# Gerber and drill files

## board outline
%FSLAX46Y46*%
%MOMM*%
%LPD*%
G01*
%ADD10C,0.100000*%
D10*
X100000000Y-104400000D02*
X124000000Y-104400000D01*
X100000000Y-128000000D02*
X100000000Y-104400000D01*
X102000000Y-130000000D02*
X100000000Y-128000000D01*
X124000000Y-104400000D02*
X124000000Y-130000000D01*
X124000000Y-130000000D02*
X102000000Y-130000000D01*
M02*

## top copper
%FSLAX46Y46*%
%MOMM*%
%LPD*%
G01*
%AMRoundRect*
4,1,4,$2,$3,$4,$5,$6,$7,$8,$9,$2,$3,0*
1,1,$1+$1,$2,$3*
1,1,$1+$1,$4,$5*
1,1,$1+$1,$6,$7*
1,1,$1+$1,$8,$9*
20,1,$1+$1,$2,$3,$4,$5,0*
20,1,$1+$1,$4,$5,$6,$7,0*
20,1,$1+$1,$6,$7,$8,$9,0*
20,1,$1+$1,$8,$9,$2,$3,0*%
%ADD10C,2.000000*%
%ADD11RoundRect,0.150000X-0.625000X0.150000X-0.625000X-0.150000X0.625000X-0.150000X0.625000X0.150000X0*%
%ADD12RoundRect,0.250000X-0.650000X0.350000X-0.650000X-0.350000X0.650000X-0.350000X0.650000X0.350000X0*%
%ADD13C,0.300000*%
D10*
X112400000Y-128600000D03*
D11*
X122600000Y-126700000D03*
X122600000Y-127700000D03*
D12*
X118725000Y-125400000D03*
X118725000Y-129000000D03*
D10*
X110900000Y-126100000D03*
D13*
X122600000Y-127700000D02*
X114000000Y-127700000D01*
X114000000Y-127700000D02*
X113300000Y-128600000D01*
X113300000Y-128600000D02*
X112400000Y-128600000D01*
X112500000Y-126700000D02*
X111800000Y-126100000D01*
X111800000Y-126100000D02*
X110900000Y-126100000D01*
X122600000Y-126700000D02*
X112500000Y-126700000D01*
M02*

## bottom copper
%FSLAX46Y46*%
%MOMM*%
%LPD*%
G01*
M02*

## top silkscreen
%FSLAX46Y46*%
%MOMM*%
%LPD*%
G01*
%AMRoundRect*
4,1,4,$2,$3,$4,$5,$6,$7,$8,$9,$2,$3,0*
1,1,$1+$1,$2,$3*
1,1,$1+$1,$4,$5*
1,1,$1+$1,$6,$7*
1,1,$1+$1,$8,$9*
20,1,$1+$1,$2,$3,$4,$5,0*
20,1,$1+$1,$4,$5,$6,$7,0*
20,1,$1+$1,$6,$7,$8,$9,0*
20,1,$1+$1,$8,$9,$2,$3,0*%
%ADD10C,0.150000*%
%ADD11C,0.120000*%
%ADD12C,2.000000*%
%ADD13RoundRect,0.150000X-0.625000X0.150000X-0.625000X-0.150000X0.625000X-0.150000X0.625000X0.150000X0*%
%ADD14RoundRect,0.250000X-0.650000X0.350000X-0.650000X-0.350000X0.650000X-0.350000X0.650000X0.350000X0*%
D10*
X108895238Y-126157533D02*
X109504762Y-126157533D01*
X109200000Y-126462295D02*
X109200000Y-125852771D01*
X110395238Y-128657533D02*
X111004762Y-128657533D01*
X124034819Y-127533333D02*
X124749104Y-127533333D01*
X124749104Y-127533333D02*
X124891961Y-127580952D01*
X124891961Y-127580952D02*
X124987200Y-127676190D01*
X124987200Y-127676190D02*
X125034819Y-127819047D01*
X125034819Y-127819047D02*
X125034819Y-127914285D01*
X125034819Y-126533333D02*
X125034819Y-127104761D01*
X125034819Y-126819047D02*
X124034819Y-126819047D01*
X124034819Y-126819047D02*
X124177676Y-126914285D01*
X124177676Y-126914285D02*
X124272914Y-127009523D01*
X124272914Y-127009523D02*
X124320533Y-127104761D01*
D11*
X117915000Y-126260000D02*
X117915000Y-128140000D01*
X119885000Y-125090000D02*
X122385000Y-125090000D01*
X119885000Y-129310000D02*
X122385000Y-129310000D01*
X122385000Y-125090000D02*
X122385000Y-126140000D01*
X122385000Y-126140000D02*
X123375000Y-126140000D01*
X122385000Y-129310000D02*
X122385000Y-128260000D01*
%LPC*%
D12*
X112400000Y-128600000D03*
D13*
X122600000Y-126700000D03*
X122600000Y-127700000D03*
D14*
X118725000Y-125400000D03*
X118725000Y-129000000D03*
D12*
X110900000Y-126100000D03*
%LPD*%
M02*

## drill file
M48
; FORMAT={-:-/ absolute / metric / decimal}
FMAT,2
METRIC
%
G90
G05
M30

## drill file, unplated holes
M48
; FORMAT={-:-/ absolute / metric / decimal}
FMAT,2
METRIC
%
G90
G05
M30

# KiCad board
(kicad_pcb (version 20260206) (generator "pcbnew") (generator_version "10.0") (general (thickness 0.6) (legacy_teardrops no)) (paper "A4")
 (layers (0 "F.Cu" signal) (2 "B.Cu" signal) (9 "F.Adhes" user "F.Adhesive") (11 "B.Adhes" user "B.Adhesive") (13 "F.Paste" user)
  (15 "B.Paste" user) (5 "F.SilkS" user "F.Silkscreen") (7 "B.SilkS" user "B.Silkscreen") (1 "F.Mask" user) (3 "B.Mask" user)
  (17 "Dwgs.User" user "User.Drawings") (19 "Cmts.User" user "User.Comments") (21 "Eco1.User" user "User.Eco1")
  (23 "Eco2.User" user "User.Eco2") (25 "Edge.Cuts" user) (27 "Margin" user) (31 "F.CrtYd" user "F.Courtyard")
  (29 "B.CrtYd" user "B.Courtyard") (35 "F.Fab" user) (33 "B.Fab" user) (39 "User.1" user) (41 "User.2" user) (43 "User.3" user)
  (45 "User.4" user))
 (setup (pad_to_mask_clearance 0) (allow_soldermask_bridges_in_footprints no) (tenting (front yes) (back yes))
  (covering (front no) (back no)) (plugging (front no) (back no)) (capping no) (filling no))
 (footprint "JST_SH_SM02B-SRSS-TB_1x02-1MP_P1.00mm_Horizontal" (layer "F.Cu") (at 120.6 127.2 -90)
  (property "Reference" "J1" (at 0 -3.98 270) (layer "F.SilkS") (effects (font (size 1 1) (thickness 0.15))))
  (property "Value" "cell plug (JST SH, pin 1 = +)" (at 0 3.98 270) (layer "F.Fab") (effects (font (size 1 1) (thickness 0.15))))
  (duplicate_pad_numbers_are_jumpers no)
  (fp_line (start -0.94 2.685) (end 0.94 2.685) (stroke (width 0.12) (type solid)) (layer "F.SilkS"))
  (fp_line (start -2.11 0.715) (end -2.11 -1.785) (stroke (width 0.12) (type solid)) (layer "F.SilkS"))
  (fp_line (start 2.11 0.715) (end 2.11 -1.785) (stroke (width 0.12) (type solid)) (layer "F.SilkS"))
  (fp_line (start -2.11 -1.785) (end -1.06 -1.785) (stroke (width 0.12) (type solid)) (layer "F.SilkS"))
  (fp_line (start -1.06 -1.785) (end -1.06 -2.775) (stroke (width 0.12) (type solid)) (layer "F.SilkS"))
  (fp_line (start 2.11 -1.785) (end 1.06 -1.785) (stroke (width 0.12) (type solid)) (layer "F.SilkS"))
  (pad "1" smd roundrect (at -0.5 -2 270) (size 0.6 1.55) (layers "F.Cu" "F.Mask" "F.Paste") (roundrect_rratio 0.25) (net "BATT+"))
  (pad "2" smd roundrect (at 0.5 -2 270) (size 0.6 1.55) (layers "F.Cu" "F.Mask" "F.Paste") (roundrect_rratio 0.25) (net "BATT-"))
  (pad "MP" smd roundrect (at -1.8 1.875 270) (size 1.2 1.8) (layers "F.Cu" "F.Mask" "F.Paste") (roundrect_rratio 0.208333))
  (pad "MP" smd roundrect (at 1.8 1.875 270) (size 1.2 1.8) (layers "F.Cu" "F.Mask" "F.Paste") (roundrect_rratio 0.208333)))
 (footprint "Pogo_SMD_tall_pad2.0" (layer "F.Cu") (at 112.4 128.6)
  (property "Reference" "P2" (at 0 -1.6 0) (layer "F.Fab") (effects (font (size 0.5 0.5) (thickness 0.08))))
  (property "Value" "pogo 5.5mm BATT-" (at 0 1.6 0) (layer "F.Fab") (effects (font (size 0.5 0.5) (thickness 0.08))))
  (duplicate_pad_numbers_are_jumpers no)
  (pad "1" smd circle (at 0 0) (size 2 2) (layers "F.Cu" "F.Mask" "F.Paste") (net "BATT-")))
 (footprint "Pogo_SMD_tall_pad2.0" (layer "F.Cu") (at 110.9 126.1)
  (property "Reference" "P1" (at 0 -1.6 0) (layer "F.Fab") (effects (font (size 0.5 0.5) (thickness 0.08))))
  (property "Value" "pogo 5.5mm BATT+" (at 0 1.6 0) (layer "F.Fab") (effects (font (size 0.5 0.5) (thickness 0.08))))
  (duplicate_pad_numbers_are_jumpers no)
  (pad "1" smd circle (at 0 0) (size 2 2) (layers "F.Cu" "F.Mask" "F.Paste") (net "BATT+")))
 (gr_line (start 100 104.4) (end 124 104.4) (stroke (width 0.1) (type default)) (layer "Edge.Cuts"))
 (gr_line (start 100 128) (end 100 104.4) (stroke (width 0.1) (type default)) (layer "Edge.Cuts"))
 (gr_line (start 102 130) (end 100 128) (stroke (width 0.1) (type default)) (layer "Edge.Cuts"))
 (gr_line (start 124 104.4) (end 124 130) (stroke (width 0.1) (type default)) (layer "Edge.Cuts"))
 (gr_line (start 124 130) (end 102 130) (stroke (width 0.1) (type default)) (layer "Edge.Cuts"))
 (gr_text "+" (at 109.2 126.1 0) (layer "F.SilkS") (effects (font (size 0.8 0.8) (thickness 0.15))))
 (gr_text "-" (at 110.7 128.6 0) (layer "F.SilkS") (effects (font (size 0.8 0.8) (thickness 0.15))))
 (segment (start 122.6 126.7) (end 112.5 126.7) (width 0.3) (layer "F.Cu") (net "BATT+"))
 (segment (start 111.8 126.1) (end 110.9 126.1) (width 0.3) (layer "F.Cu") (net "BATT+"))
 (segment (start 112.5 126.7) (end 111.8 126.1) (width 0.3) (layer "F.Cu") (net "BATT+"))
 (segment (start 114 127.7) (end 113.3 128.6) (width 0.3) (layer "F.Cu") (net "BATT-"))
 (segment (start 122.6 127.7) (end 114 127.7) (width 0.3) (layer "F.Cu") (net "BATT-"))
 (segment (start 113.3 128.6) (end 112.4 128.6) (width 0.3) (layer "F.Cu") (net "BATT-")))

